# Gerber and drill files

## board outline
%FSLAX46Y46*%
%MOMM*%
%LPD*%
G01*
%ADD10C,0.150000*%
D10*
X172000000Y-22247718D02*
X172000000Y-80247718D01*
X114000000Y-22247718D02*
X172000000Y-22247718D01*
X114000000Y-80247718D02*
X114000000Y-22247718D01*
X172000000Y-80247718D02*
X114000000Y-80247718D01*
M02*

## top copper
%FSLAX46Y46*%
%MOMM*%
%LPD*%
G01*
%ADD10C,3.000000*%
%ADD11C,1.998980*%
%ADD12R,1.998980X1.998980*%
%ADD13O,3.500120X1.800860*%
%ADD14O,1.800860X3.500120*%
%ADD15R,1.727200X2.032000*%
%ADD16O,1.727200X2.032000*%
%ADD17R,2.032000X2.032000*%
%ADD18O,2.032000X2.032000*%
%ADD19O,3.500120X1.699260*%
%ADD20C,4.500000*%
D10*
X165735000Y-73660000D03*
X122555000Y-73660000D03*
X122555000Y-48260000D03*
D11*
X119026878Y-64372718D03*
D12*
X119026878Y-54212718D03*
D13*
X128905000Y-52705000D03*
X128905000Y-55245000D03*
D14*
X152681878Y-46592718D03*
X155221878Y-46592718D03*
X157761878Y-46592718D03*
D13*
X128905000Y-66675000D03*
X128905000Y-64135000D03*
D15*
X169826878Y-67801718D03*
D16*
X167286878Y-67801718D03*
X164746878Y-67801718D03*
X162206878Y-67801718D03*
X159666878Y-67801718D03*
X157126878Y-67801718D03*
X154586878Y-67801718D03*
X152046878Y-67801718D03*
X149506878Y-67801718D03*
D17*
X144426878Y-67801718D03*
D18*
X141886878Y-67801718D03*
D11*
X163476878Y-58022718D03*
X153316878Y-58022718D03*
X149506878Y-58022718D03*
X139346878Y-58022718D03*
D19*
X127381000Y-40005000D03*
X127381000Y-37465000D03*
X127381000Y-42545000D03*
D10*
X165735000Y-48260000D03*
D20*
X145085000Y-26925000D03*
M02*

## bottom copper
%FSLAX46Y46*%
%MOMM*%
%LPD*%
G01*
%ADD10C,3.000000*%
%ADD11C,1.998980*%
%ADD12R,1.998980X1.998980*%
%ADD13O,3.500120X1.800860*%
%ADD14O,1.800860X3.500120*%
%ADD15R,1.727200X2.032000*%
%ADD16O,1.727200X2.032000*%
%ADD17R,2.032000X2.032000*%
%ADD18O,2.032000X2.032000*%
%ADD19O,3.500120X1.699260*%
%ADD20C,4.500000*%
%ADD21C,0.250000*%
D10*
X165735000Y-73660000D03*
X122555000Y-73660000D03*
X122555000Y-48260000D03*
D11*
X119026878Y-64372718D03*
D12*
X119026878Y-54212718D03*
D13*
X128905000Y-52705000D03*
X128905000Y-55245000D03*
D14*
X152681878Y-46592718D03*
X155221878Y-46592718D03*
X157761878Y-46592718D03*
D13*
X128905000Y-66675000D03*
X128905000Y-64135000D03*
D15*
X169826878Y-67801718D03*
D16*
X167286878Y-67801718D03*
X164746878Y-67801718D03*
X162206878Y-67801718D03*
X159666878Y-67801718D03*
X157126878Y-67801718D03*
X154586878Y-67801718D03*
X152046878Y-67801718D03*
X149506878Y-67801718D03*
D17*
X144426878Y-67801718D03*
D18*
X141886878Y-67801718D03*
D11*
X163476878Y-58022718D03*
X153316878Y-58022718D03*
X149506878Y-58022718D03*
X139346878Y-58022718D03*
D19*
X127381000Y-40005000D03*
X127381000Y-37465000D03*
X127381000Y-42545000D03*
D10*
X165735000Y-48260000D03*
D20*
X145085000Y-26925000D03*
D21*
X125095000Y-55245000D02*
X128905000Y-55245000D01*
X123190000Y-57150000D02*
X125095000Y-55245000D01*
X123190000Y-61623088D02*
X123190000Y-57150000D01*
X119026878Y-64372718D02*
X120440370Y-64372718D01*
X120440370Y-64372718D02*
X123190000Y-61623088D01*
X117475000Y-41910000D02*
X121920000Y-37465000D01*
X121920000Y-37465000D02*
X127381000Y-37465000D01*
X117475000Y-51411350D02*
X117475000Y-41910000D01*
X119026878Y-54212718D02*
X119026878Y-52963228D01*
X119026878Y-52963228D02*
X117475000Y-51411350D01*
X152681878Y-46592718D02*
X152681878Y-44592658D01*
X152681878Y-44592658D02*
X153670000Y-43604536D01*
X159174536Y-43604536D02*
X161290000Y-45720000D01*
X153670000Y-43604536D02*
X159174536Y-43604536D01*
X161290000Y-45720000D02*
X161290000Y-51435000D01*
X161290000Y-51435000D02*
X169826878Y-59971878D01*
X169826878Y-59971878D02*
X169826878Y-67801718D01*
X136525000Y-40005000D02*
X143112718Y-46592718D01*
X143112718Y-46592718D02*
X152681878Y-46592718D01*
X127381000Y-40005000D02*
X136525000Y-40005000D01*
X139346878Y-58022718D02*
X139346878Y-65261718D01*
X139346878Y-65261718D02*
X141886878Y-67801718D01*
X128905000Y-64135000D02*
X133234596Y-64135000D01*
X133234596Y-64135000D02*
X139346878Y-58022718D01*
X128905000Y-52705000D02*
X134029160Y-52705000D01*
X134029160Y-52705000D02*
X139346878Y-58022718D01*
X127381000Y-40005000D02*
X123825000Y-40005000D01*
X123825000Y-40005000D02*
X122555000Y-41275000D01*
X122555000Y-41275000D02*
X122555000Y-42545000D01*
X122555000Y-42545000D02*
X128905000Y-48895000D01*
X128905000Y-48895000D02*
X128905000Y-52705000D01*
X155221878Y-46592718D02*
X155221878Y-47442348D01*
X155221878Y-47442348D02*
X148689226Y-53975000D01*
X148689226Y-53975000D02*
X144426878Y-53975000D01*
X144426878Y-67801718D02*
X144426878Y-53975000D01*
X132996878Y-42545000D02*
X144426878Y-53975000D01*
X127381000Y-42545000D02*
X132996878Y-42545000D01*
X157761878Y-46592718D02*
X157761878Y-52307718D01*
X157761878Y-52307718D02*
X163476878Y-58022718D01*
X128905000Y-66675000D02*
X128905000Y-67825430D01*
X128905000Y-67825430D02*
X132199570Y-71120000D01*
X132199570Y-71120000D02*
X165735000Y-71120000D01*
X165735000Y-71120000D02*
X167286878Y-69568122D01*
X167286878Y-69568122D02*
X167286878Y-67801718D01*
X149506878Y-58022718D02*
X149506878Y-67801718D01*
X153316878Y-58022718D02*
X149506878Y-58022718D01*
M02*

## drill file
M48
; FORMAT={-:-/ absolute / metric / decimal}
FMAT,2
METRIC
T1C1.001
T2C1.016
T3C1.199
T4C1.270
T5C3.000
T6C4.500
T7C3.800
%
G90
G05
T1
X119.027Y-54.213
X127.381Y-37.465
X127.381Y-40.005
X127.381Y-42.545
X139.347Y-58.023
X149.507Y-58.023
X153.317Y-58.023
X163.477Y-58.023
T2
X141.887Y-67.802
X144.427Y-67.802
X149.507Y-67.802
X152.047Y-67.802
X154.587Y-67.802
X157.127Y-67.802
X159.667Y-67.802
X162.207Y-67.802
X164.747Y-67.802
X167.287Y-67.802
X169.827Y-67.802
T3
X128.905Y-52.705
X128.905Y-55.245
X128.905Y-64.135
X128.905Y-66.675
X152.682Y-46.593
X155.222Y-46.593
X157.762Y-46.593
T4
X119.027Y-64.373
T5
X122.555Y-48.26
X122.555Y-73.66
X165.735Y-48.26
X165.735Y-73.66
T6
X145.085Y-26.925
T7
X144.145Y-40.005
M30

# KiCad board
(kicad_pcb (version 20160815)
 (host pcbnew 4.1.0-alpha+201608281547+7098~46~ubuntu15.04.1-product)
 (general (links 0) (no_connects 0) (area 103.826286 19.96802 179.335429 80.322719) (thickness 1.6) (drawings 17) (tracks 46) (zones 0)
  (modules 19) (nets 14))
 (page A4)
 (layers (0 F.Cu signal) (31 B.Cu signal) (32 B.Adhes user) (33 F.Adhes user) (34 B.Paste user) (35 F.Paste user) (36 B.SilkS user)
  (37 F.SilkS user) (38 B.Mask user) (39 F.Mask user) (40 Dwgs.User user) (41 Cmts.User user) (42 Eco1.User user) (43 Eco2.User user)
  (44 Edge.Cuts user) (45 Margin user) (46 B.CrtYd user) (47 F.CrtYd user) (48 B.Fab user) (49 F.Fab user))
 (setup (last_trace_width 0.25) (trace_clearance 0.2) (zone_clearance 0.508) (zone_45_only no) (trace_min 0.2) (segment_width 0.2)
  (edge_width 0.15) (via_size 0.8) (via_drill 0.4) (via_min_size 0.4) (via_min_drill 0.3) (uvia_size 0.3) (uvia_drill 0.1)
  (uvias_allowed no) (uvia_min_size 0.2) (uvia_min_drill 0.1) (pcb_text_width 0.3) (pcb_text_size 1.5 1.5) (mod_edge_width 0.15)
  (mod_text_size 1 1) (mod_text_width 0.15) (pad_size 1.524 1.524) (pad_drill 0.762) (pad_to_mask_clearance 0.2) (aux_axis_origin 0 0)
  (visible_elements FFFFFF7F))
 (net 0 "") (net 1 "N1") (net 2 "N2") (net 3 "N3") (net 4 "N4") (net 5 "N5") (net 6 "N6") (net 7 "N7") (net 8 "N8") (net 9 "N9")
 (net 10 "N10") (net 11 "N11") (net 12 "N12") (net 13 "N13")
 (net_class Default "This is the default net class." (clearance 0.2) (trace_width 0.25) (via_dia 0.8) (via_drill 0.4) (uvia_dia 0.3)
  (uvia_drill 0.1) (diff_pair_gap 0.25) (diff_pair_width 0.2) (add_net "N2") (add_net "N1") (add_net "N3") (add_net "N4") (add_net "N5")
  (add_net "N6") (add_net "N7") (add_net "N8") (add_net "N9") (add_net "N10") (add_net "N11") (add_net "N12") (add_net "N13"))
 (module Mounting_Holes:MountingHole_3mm (layer F.Cu) (at 165.735 73.66)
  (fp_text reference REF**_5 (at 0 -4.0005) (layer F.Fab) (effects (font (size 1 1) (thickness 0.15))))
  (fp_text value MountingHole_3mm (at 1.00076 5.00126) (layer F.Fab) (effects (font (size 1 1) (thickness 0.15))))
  (pad 1 thru_hole circle (at 0 0) (size 3 3) (drill 3)))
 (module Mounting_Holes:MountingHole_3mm (layer F.Cu) (at 122.555 73.66)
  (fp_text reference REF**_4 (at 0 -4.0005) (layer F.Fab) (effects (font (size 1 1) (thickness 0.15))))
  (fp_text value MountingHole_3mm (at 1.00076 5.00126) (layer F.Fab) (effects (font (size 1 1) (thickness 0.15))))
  (pad 1 thru_hole circle (at 0 0) (size 3 3) (drill 3)))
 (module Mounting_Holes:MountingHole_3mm (layer F.Cu) (at 122.555 48.26)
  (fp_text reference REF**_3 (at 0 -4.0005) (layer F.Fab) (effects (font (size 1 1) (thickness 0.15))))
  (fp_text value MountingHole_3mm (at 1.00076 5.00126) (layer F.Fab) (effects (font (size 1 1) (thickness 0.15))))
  (pad 1 thru_hole circle (at 0 0) (size 3 3) (drill 3)))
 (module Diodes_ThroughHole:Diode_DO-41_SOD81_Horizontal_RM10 (layer F.Cu) (at 119.024338 54.212718 270)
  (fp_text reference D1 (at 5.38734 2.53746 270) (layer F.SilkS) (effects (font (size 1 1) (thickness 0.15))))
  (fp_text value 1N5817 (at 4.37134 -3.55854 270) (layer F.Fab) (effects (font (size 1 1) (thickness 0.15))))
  (pad 2 thru_hole circle (at 10.16 -0.00254 90) (size 1.99898 1.99898) (drill 1.27) (layers *.Cu *.Mask F.SilkS) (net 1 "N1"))
  (pad 1 thru_hole rect (at 0 -0.00254 90) (size 1.99898 1.99898) (drill 1.00076) (layers *.Cu *.Mask F.SilkS) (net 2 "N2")))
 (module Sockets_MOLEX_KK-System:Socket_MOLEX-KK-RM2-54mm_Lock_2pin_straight (layer F.Cu) (at 128.905 53.975 270)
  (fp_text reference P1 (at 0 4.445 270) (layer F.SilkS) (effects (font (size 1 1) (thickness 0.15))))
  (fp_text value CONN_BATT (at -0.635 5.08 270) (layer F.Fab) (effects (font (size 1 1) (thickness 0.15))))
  (pad 1 thru_hole oval (at -1.27 0 270) (size 1.80086 3.50012) (drill 1.19888) (layers *.Cu *.Mask F.SilkS) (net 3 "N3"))
  (pad 2 thru_hole oval (at 1.27 0 270) (size 1.80086 3.50012) (drill 1.19888) (layers *.Cu *.Mask F.SilkS) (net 1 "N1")))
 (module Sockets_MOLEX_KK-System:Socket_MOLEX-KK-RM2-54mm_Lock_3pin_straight (layer F.Cu) (at 155.221878 46.592718)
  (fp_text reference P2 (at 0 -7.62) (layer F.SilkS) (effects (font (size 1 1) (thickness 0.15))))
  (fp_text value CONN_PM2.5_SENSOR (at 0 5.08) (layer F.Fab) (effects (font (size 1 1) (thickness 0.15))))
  (pad 1 thru_hole oval (at -2.54 0) (size 1.80086 3.50012) (drill 1.19888) (layers *.Cu *.Mask F.SilkS) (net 3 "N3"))
  (pad 2 thru_hole oval (at 0 0) (size 1.80086 3.50012) (drill 1.19888) (layers *.Cu *.Mask F.SilkS) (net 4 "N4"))
  (pad 3 thru_hole oval (at 2.54 0) (size 1.80086 3.50012) (drill 1.19888) (layers *.Cu *.Mask F.SilkS) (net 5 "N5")))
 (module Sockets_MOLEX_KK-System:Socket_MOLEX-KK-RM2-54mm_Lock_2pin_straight (layer F.Cu) (at 128.905 65.405 90)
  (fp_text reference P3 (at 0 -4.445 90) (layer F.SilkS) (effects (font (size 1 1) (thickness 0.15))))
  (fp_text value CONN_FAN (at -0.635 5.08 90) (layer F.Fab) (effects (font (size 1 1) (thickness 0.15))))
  (pad 1 thru_hole oval (at -1.27 0 90) (size 1.80086 3.50012) (drill 1.19888) (layers *.Cu *.Mask F.SilkS) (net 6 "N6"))
  (pad 2 thru_hole oval (at 1.27 0 90) (size 1.80086 3.50012) (drill 1.19888) (layers *.Cu *.Mask F.SilkS) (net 3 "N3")))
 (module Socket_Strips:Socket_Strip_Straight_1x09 (layer F.Cu) (at 169.826878 67.801718 180)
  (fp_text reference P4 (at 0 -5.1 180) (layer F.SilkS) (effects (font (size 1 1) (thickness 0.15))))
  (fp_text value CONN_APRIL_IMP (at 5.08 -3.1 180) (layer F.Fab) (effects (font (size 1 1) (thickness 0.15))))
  (pad 1 thru_hole rect (at 0 0 180) (size 1.7272 2.032) (drill 1.016) (layers *.Cu *.Mask F.SilkS) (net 3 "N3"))
  (pad 2 thru_hole oval (at 2.54 0 180) (size 1.7272 2.032) (drill 1.016) (layers *.Cu *.Mask F.SilkS) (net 6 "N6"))
  (pad 3 thru_hole oval (at 5.08 0 180) (size 1.7272 2.032) (drill 1.016) (layers *.Cu *.Mask F.SilkS) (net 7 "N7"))
  (pad 4 thru_hole oval (at 7.62 0 180) (size 1.7272 2.032) (drill 1.016) (layers *.Cu *.Mask F.SilkS) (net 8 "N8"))
  (pad 5 thru_hole oval (at 10.16 0 180) (size 1.7272 2.032) (drill 1.016) (layers *.Cu *.Mask F.SilkS) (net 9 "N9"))
  (pad 6 thru_hole oval (at 12.7 0 180) (size 1.7272 2.032) (drill 1.016) (layers *.Cu *.Mask F.SilkS) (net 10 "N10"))
  (pad 7 thru_hole oval (at 15.24 0 180) (size 1.7272 2.032) (drill 1.016) (layers *.Cu *.Mask F.SilkS) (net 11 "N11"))
  (pad 8 thru_hole oval (at 17.78 0 180) (size 1.7272 2.032) (drill 1.016) (layers *.Cu *.Mask F.SilkS) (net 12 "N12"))
  (pad 9 thru_hole oval (at 20.32 0 180) (size 1.7272 2.032) (drill 1.016) (layers *.Cu *.Mask F.SilkS) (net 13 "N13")))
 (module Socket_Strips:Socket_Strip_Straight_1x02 (layer F.Cu) (at 144.426878 67.801718 180)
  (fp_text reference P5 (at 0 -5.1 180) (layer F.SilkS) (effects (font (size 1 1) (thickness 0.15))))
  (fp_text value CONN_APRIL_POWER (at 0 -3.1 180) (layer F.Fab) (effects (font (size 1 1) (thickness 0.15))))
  (pad 1 thru_hole rect (at 0 0 180) (size 2.032 2.032) (drill 1.016) (layers *.Cu *.Mask F.SilkS) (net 4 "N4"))
  (pad 2 thru_hole oval (at 2.54 0 180) (size 2.032 2.032) (drill 1.016) (layers *.Cu *.Mask F.SilkS) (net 3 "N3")))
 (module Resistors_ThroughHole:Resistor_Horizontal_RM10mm (layer F.Cu) (at 158.396878 58.022718 180)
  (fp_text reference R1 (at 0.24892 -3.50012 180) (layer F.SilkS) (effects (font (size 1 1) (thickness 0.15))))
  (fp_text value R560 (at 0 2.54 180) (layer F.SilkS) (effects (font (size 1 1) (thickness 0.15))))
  (pad 1 thru_hole circle (at -5.08 0 180) (size 1.99898 1.99898) (drill 1.00076) (layers *.Cu *.SilkS *.Mask) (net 5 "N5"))
  (pad 2 thru_hole circle (at 5.08 0 180) (size 1.99898 1.99898) (drill 1.00076) (layers *.Cu *.SilkS *.Mask) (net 13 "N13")))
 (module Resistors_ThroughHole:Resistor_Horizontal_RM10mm (layer F.Cu) (at 144.426878 58.022718 180)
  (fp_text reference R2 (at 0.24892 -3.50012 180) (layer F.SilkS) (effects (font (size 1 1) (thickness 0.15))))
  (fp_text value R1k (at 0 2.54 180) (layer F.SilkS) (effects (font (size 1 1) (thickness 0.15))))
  (pad 1 thru_hole circle (at -5.08 0 180) (size 1.99898 1.99898) (drill 1.00076) (layers *.Cu *.SilkS *.Mask) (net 13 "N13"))
  (pad 2 thru_hole circle (at 5.08 0 180) (size 1.99898 1.99898) (drill 1.00076) (layers *.Cu *.SilkS *.Mask) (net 3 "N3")))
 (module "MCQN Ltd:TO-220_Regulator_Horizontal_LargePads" (layer F.Cu) (at 127.381 40.005 270)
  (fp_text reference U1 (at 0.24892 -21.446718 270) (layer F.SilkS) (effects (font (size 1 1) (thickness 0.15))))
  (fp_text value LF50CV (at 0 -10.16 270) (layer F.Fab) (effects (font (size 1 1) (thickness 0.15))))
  (pad GND thru_hole oval (at 0 0) (size 3.50012 1.69926) (drill 1.00076) (layers *.Cu *.Mask F.SilkS) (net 3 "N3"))
  (pad VI thru_hole oval (at -2.54 0) (size 3.50012 1.69926) (drill 1.00076) (layers *.Cu *.Mask F.SilkS) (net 2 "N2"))
  (pad VO thru_hole oval (at 2.54 0) (size 3.50012 1.69926) (drill 1.00076) (layers *.Cu *.Mask F.SilkS) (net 4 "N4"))
  (pad "" np_thru_hole circle (at 0 -16.764) (size 3.79984 3.79984) (drill 3.79984) (layers *.Cu *.Mask F.SilkS)))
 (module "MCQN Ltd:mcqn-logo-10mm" (layer F.Cu) (at 165.487038 27.760574)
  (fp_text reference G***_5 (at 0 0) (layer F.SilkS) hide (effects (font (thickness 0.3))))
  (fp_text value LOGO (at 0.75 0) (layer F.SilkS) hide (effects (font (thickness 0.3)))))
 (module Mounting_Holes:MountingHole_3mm (layer F.Cu) (at 165.735 48.26)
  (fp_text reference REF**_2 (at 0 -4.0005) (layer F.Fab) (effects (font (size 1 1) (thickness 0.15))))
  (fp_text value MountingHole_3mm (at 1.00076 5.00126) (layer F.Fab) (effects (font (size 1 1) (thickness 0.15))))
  (pad 1 thru_hole circle (at 0 0) (size 3 3) (drill 3)))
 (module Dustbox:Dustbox (layer F.Cu) (at 175.26 35.56)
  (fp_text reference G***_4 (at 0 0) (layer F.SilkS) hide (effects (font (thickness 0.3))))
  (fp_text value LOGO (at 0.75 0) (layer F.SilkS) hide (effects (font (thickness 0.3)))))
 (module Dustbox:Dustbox (layer F.Cu) (at 106.68 29.21)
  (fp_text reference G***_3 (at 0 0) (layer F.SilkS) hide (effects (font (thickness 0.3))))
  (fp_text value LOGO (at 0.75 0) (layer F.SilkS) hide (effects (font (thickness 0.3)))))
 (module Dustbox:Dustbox (layer F.Cu) (at 126.365 26.035)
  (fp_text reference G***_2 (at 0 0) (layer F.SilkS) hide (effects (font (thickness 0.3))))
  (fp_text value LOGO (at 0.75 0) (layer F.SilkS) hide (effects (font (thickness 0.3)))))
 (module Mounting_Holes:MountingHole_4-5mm (layer F.Cu) (at 145.085 26.925)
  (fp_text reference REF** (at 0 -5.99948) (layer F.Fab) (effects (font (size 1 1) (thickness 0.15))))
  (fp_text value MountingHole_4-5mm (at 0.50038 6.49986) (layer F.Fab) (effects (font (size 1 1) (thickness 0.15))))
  (pad 1 thru_hole circle (at 0 0) (size 4.5 4.5) (drill 4.5)))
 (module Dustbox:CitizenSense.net (layer F.Cu) (at 126.238 29.718)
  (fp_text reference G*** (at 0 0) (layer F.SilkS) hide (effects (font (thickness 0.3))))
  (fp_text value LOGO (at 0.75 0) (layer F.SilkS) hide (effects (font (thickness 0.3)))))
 (gr_line (start 172 22.247718) (end 172 80.247718) (layer Edge.Cuts) (width 0.15))
 (gr_line (start 114 22.247718) (end 172 22.247718) (layer Edge.Cuts) (width 0.15))
 (gr_line (start 114 80.247718) (end 114 22.247718) (layer Edge.Cuts) (width 0.15))
 (gr_line (start 172 80.247718) (end 114 80.247718) (layer Edge.Cuts) (width 0.15))
 (segment (start 125.095 55.245) (end 128.905 55.245) (width 0.25) (layer B.Cu) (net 1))
 (segment (start 123.19 57.15) (end 125.095 55.245) (width 0.25) (layer B.Cu) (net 1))
 (segment (start 123.19 61.623088) (end 123.19 57.15) (width 0.25) (layer B.Cu) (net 1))
 (segment (start 119.026878 64.372718) (end 120.44037 64.372718) (width 0.25) (layer B.Cu) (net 1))
 (segment (start 120.44037 64.372718) (end 123.19 61.623088) (width 0.25) (layer B.Cu) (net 1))
 (segment (start 117.475 41.91) (end 121.92 37.465) (width 0.25) (layer B.Cu) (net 2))
 (segment (start 121.92 37.465) (end 127.381 37.465) (width 0.25) (layer B.Cu) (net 2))
 (segment (start 117.475 51.41135) (end 117.475 41.91) (width 0.25) (layer B.Cu) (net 2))
 (segment (start 119.026878 54.212718) (end 119.026878 52.963228) (width 0.25) (layer B.Cu) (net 2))
 (segment (start 119.026878 52.963228) (end 117.475 51.41135) (width 0.25) (layer B.Cu) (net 2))
 (segment (start 152.681878 46.592718) (end 152.681878 44.592658) (width 0.25) (layer B.Cu) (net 3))
 (segment (start 152.681878 44.592658) (end 153.67 43.604536) (width 0.25) (layer B.Cu) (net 3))
 (segment (start 159.174536 43.604536) (end 161.29 45.72) (width 0.25) (layer B.Cu) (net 3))
 (segment (start 153.67 43.604536) (end 159.174536 43.604536) (width 0.25) (layer B.Cu) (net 3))
 (segment (start 161.29 45.72) (end 161.29 51.435) (width 0.25) (layer B.Cu) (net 3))
 (segment (start 161.29 51.435) (end 169.826878 59.971878) (width 0.25) (layer B.Cu) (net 3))
 (segment (start 169.826878 59.971878) (end 169.826878 67.801718) (width 0.25) (layer B.Cu) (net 3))
 (segment (start 136.525 40.005) (end 143.112718 46.592718) (width 0.25) (layer B.Cu) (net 3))
 (segment (start 143.112718 46.592718) (end 152.681878 46.592718) (width 0.25) (layer B.Cu) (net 3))
 (segment (start 127.381 40.005) (end 136.525 40.005) (width 0.25) (layer B.Cu) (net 3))
 (segment (start 139.346878 58.022718) (end 139.346878 65.261718) (width 0.25) (layer B.Cu) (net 3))
 (segment (start 139.346878 65.261718) (end 141.886878 67.801718) (width 0.25) (layer B.Cu) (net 3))
 (segment (start 128.905 64.135) (end 133.234596 64.135) (width 0.25) (layer B.Cu) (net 3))
 (segment (start 133.234596 64.135) (end 139.346878 58.022718) (width 0.25) (layer B.Cu) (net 3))
 (segment (start 128.905 52.705) (end 134.02916 52.705) (width 0.25) (layer B.Cu) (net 3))
 (segment (start 134.02916 52.705) (end 139.346878 58.022718) (width 0.25) (layer B.Cu) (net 3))
 (segment (start 127.381 40.005) (end 123.825 40.005) (width 0.25) (layer B.Cu) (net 3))
 (segment (start 123.825 40.005) (end 122.555 41.275) (width 0.25) (layer B.Cu) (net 3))
 (segment (start 122.555 41.275) (end 122.555 42.545) (width 0.25) (layer B.Cu) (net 3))
 (segment (start 122.555 42.545) (end 128.905 48.895) (width 0.25) (layer B.Cu) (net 3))
 (segment (start 128.905 48.895) (end 128.905 52.705) (width 0.25) (layer B.Cu) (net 3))
 (segment (start 155.221878 46.592718) (end 155.221878 47.442348) (width 0.25) (layer B.Cu) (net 4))
 (segment (start 155.221878 47.442348) (end 148.689226 53.975) (width 0.25) (layer B.Cu) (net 4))
 (segment (start 148.689226 53.975) (end 144.426878 53.975) (width 0.25) (layer B.Cu) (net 4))
 (segment (start 144.426878 67.801718) (end 144.426878 53.975) (width 0.25) (layer B.Cu) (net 4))
 (segment (start 132.996878 42.545) (end 144.426878 53.975) (width 0.25) (layer B.Cu) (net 4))
 (segment (start 127.381 42.545) (end 132.996878 42.545) (width 0.25) (layer B.Cu) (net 4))
 (segment (start 157.761878 46.592718) (end 157.761878 52.307718) (width 0.25) (layer B.Cu) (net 5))
 (segment (start 157.761878 52.307718) (end 163.476878 58.022718) (width 0.25) (layer B.Cu) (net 5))
 (segment (start 128.905 66.675) (end 128.905 67.82543) (width 0.25) (layer B.Cu) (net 6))
 (segment (start 128.905 67.82543) (end 132.19957 71.12) (width 0.25) (layer B.Cu) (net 6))
 (segment (start 132.19957 71.12) (end 165.735 71.12) (width 0.25) (layer B.Cu) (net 6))
 (segment (start 165.735 71.12) (end 167.286878 69.568122) (width 0.25) (layer B.Cu) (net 6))
 (segment (start 167.286878 69.568122) (end 167.286878 67.801718) (width 0.25) (layer B.Cu) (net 6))
 (segment (start 149.506878 58.022718) (end 149.506878 67.801718) (width 0.25) (layer B.Cu) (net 13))
 (segment (start 153.316878 58.022718) (end 149.506878 58.022718) (width 0.25) (layer B.Cu) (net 13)))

